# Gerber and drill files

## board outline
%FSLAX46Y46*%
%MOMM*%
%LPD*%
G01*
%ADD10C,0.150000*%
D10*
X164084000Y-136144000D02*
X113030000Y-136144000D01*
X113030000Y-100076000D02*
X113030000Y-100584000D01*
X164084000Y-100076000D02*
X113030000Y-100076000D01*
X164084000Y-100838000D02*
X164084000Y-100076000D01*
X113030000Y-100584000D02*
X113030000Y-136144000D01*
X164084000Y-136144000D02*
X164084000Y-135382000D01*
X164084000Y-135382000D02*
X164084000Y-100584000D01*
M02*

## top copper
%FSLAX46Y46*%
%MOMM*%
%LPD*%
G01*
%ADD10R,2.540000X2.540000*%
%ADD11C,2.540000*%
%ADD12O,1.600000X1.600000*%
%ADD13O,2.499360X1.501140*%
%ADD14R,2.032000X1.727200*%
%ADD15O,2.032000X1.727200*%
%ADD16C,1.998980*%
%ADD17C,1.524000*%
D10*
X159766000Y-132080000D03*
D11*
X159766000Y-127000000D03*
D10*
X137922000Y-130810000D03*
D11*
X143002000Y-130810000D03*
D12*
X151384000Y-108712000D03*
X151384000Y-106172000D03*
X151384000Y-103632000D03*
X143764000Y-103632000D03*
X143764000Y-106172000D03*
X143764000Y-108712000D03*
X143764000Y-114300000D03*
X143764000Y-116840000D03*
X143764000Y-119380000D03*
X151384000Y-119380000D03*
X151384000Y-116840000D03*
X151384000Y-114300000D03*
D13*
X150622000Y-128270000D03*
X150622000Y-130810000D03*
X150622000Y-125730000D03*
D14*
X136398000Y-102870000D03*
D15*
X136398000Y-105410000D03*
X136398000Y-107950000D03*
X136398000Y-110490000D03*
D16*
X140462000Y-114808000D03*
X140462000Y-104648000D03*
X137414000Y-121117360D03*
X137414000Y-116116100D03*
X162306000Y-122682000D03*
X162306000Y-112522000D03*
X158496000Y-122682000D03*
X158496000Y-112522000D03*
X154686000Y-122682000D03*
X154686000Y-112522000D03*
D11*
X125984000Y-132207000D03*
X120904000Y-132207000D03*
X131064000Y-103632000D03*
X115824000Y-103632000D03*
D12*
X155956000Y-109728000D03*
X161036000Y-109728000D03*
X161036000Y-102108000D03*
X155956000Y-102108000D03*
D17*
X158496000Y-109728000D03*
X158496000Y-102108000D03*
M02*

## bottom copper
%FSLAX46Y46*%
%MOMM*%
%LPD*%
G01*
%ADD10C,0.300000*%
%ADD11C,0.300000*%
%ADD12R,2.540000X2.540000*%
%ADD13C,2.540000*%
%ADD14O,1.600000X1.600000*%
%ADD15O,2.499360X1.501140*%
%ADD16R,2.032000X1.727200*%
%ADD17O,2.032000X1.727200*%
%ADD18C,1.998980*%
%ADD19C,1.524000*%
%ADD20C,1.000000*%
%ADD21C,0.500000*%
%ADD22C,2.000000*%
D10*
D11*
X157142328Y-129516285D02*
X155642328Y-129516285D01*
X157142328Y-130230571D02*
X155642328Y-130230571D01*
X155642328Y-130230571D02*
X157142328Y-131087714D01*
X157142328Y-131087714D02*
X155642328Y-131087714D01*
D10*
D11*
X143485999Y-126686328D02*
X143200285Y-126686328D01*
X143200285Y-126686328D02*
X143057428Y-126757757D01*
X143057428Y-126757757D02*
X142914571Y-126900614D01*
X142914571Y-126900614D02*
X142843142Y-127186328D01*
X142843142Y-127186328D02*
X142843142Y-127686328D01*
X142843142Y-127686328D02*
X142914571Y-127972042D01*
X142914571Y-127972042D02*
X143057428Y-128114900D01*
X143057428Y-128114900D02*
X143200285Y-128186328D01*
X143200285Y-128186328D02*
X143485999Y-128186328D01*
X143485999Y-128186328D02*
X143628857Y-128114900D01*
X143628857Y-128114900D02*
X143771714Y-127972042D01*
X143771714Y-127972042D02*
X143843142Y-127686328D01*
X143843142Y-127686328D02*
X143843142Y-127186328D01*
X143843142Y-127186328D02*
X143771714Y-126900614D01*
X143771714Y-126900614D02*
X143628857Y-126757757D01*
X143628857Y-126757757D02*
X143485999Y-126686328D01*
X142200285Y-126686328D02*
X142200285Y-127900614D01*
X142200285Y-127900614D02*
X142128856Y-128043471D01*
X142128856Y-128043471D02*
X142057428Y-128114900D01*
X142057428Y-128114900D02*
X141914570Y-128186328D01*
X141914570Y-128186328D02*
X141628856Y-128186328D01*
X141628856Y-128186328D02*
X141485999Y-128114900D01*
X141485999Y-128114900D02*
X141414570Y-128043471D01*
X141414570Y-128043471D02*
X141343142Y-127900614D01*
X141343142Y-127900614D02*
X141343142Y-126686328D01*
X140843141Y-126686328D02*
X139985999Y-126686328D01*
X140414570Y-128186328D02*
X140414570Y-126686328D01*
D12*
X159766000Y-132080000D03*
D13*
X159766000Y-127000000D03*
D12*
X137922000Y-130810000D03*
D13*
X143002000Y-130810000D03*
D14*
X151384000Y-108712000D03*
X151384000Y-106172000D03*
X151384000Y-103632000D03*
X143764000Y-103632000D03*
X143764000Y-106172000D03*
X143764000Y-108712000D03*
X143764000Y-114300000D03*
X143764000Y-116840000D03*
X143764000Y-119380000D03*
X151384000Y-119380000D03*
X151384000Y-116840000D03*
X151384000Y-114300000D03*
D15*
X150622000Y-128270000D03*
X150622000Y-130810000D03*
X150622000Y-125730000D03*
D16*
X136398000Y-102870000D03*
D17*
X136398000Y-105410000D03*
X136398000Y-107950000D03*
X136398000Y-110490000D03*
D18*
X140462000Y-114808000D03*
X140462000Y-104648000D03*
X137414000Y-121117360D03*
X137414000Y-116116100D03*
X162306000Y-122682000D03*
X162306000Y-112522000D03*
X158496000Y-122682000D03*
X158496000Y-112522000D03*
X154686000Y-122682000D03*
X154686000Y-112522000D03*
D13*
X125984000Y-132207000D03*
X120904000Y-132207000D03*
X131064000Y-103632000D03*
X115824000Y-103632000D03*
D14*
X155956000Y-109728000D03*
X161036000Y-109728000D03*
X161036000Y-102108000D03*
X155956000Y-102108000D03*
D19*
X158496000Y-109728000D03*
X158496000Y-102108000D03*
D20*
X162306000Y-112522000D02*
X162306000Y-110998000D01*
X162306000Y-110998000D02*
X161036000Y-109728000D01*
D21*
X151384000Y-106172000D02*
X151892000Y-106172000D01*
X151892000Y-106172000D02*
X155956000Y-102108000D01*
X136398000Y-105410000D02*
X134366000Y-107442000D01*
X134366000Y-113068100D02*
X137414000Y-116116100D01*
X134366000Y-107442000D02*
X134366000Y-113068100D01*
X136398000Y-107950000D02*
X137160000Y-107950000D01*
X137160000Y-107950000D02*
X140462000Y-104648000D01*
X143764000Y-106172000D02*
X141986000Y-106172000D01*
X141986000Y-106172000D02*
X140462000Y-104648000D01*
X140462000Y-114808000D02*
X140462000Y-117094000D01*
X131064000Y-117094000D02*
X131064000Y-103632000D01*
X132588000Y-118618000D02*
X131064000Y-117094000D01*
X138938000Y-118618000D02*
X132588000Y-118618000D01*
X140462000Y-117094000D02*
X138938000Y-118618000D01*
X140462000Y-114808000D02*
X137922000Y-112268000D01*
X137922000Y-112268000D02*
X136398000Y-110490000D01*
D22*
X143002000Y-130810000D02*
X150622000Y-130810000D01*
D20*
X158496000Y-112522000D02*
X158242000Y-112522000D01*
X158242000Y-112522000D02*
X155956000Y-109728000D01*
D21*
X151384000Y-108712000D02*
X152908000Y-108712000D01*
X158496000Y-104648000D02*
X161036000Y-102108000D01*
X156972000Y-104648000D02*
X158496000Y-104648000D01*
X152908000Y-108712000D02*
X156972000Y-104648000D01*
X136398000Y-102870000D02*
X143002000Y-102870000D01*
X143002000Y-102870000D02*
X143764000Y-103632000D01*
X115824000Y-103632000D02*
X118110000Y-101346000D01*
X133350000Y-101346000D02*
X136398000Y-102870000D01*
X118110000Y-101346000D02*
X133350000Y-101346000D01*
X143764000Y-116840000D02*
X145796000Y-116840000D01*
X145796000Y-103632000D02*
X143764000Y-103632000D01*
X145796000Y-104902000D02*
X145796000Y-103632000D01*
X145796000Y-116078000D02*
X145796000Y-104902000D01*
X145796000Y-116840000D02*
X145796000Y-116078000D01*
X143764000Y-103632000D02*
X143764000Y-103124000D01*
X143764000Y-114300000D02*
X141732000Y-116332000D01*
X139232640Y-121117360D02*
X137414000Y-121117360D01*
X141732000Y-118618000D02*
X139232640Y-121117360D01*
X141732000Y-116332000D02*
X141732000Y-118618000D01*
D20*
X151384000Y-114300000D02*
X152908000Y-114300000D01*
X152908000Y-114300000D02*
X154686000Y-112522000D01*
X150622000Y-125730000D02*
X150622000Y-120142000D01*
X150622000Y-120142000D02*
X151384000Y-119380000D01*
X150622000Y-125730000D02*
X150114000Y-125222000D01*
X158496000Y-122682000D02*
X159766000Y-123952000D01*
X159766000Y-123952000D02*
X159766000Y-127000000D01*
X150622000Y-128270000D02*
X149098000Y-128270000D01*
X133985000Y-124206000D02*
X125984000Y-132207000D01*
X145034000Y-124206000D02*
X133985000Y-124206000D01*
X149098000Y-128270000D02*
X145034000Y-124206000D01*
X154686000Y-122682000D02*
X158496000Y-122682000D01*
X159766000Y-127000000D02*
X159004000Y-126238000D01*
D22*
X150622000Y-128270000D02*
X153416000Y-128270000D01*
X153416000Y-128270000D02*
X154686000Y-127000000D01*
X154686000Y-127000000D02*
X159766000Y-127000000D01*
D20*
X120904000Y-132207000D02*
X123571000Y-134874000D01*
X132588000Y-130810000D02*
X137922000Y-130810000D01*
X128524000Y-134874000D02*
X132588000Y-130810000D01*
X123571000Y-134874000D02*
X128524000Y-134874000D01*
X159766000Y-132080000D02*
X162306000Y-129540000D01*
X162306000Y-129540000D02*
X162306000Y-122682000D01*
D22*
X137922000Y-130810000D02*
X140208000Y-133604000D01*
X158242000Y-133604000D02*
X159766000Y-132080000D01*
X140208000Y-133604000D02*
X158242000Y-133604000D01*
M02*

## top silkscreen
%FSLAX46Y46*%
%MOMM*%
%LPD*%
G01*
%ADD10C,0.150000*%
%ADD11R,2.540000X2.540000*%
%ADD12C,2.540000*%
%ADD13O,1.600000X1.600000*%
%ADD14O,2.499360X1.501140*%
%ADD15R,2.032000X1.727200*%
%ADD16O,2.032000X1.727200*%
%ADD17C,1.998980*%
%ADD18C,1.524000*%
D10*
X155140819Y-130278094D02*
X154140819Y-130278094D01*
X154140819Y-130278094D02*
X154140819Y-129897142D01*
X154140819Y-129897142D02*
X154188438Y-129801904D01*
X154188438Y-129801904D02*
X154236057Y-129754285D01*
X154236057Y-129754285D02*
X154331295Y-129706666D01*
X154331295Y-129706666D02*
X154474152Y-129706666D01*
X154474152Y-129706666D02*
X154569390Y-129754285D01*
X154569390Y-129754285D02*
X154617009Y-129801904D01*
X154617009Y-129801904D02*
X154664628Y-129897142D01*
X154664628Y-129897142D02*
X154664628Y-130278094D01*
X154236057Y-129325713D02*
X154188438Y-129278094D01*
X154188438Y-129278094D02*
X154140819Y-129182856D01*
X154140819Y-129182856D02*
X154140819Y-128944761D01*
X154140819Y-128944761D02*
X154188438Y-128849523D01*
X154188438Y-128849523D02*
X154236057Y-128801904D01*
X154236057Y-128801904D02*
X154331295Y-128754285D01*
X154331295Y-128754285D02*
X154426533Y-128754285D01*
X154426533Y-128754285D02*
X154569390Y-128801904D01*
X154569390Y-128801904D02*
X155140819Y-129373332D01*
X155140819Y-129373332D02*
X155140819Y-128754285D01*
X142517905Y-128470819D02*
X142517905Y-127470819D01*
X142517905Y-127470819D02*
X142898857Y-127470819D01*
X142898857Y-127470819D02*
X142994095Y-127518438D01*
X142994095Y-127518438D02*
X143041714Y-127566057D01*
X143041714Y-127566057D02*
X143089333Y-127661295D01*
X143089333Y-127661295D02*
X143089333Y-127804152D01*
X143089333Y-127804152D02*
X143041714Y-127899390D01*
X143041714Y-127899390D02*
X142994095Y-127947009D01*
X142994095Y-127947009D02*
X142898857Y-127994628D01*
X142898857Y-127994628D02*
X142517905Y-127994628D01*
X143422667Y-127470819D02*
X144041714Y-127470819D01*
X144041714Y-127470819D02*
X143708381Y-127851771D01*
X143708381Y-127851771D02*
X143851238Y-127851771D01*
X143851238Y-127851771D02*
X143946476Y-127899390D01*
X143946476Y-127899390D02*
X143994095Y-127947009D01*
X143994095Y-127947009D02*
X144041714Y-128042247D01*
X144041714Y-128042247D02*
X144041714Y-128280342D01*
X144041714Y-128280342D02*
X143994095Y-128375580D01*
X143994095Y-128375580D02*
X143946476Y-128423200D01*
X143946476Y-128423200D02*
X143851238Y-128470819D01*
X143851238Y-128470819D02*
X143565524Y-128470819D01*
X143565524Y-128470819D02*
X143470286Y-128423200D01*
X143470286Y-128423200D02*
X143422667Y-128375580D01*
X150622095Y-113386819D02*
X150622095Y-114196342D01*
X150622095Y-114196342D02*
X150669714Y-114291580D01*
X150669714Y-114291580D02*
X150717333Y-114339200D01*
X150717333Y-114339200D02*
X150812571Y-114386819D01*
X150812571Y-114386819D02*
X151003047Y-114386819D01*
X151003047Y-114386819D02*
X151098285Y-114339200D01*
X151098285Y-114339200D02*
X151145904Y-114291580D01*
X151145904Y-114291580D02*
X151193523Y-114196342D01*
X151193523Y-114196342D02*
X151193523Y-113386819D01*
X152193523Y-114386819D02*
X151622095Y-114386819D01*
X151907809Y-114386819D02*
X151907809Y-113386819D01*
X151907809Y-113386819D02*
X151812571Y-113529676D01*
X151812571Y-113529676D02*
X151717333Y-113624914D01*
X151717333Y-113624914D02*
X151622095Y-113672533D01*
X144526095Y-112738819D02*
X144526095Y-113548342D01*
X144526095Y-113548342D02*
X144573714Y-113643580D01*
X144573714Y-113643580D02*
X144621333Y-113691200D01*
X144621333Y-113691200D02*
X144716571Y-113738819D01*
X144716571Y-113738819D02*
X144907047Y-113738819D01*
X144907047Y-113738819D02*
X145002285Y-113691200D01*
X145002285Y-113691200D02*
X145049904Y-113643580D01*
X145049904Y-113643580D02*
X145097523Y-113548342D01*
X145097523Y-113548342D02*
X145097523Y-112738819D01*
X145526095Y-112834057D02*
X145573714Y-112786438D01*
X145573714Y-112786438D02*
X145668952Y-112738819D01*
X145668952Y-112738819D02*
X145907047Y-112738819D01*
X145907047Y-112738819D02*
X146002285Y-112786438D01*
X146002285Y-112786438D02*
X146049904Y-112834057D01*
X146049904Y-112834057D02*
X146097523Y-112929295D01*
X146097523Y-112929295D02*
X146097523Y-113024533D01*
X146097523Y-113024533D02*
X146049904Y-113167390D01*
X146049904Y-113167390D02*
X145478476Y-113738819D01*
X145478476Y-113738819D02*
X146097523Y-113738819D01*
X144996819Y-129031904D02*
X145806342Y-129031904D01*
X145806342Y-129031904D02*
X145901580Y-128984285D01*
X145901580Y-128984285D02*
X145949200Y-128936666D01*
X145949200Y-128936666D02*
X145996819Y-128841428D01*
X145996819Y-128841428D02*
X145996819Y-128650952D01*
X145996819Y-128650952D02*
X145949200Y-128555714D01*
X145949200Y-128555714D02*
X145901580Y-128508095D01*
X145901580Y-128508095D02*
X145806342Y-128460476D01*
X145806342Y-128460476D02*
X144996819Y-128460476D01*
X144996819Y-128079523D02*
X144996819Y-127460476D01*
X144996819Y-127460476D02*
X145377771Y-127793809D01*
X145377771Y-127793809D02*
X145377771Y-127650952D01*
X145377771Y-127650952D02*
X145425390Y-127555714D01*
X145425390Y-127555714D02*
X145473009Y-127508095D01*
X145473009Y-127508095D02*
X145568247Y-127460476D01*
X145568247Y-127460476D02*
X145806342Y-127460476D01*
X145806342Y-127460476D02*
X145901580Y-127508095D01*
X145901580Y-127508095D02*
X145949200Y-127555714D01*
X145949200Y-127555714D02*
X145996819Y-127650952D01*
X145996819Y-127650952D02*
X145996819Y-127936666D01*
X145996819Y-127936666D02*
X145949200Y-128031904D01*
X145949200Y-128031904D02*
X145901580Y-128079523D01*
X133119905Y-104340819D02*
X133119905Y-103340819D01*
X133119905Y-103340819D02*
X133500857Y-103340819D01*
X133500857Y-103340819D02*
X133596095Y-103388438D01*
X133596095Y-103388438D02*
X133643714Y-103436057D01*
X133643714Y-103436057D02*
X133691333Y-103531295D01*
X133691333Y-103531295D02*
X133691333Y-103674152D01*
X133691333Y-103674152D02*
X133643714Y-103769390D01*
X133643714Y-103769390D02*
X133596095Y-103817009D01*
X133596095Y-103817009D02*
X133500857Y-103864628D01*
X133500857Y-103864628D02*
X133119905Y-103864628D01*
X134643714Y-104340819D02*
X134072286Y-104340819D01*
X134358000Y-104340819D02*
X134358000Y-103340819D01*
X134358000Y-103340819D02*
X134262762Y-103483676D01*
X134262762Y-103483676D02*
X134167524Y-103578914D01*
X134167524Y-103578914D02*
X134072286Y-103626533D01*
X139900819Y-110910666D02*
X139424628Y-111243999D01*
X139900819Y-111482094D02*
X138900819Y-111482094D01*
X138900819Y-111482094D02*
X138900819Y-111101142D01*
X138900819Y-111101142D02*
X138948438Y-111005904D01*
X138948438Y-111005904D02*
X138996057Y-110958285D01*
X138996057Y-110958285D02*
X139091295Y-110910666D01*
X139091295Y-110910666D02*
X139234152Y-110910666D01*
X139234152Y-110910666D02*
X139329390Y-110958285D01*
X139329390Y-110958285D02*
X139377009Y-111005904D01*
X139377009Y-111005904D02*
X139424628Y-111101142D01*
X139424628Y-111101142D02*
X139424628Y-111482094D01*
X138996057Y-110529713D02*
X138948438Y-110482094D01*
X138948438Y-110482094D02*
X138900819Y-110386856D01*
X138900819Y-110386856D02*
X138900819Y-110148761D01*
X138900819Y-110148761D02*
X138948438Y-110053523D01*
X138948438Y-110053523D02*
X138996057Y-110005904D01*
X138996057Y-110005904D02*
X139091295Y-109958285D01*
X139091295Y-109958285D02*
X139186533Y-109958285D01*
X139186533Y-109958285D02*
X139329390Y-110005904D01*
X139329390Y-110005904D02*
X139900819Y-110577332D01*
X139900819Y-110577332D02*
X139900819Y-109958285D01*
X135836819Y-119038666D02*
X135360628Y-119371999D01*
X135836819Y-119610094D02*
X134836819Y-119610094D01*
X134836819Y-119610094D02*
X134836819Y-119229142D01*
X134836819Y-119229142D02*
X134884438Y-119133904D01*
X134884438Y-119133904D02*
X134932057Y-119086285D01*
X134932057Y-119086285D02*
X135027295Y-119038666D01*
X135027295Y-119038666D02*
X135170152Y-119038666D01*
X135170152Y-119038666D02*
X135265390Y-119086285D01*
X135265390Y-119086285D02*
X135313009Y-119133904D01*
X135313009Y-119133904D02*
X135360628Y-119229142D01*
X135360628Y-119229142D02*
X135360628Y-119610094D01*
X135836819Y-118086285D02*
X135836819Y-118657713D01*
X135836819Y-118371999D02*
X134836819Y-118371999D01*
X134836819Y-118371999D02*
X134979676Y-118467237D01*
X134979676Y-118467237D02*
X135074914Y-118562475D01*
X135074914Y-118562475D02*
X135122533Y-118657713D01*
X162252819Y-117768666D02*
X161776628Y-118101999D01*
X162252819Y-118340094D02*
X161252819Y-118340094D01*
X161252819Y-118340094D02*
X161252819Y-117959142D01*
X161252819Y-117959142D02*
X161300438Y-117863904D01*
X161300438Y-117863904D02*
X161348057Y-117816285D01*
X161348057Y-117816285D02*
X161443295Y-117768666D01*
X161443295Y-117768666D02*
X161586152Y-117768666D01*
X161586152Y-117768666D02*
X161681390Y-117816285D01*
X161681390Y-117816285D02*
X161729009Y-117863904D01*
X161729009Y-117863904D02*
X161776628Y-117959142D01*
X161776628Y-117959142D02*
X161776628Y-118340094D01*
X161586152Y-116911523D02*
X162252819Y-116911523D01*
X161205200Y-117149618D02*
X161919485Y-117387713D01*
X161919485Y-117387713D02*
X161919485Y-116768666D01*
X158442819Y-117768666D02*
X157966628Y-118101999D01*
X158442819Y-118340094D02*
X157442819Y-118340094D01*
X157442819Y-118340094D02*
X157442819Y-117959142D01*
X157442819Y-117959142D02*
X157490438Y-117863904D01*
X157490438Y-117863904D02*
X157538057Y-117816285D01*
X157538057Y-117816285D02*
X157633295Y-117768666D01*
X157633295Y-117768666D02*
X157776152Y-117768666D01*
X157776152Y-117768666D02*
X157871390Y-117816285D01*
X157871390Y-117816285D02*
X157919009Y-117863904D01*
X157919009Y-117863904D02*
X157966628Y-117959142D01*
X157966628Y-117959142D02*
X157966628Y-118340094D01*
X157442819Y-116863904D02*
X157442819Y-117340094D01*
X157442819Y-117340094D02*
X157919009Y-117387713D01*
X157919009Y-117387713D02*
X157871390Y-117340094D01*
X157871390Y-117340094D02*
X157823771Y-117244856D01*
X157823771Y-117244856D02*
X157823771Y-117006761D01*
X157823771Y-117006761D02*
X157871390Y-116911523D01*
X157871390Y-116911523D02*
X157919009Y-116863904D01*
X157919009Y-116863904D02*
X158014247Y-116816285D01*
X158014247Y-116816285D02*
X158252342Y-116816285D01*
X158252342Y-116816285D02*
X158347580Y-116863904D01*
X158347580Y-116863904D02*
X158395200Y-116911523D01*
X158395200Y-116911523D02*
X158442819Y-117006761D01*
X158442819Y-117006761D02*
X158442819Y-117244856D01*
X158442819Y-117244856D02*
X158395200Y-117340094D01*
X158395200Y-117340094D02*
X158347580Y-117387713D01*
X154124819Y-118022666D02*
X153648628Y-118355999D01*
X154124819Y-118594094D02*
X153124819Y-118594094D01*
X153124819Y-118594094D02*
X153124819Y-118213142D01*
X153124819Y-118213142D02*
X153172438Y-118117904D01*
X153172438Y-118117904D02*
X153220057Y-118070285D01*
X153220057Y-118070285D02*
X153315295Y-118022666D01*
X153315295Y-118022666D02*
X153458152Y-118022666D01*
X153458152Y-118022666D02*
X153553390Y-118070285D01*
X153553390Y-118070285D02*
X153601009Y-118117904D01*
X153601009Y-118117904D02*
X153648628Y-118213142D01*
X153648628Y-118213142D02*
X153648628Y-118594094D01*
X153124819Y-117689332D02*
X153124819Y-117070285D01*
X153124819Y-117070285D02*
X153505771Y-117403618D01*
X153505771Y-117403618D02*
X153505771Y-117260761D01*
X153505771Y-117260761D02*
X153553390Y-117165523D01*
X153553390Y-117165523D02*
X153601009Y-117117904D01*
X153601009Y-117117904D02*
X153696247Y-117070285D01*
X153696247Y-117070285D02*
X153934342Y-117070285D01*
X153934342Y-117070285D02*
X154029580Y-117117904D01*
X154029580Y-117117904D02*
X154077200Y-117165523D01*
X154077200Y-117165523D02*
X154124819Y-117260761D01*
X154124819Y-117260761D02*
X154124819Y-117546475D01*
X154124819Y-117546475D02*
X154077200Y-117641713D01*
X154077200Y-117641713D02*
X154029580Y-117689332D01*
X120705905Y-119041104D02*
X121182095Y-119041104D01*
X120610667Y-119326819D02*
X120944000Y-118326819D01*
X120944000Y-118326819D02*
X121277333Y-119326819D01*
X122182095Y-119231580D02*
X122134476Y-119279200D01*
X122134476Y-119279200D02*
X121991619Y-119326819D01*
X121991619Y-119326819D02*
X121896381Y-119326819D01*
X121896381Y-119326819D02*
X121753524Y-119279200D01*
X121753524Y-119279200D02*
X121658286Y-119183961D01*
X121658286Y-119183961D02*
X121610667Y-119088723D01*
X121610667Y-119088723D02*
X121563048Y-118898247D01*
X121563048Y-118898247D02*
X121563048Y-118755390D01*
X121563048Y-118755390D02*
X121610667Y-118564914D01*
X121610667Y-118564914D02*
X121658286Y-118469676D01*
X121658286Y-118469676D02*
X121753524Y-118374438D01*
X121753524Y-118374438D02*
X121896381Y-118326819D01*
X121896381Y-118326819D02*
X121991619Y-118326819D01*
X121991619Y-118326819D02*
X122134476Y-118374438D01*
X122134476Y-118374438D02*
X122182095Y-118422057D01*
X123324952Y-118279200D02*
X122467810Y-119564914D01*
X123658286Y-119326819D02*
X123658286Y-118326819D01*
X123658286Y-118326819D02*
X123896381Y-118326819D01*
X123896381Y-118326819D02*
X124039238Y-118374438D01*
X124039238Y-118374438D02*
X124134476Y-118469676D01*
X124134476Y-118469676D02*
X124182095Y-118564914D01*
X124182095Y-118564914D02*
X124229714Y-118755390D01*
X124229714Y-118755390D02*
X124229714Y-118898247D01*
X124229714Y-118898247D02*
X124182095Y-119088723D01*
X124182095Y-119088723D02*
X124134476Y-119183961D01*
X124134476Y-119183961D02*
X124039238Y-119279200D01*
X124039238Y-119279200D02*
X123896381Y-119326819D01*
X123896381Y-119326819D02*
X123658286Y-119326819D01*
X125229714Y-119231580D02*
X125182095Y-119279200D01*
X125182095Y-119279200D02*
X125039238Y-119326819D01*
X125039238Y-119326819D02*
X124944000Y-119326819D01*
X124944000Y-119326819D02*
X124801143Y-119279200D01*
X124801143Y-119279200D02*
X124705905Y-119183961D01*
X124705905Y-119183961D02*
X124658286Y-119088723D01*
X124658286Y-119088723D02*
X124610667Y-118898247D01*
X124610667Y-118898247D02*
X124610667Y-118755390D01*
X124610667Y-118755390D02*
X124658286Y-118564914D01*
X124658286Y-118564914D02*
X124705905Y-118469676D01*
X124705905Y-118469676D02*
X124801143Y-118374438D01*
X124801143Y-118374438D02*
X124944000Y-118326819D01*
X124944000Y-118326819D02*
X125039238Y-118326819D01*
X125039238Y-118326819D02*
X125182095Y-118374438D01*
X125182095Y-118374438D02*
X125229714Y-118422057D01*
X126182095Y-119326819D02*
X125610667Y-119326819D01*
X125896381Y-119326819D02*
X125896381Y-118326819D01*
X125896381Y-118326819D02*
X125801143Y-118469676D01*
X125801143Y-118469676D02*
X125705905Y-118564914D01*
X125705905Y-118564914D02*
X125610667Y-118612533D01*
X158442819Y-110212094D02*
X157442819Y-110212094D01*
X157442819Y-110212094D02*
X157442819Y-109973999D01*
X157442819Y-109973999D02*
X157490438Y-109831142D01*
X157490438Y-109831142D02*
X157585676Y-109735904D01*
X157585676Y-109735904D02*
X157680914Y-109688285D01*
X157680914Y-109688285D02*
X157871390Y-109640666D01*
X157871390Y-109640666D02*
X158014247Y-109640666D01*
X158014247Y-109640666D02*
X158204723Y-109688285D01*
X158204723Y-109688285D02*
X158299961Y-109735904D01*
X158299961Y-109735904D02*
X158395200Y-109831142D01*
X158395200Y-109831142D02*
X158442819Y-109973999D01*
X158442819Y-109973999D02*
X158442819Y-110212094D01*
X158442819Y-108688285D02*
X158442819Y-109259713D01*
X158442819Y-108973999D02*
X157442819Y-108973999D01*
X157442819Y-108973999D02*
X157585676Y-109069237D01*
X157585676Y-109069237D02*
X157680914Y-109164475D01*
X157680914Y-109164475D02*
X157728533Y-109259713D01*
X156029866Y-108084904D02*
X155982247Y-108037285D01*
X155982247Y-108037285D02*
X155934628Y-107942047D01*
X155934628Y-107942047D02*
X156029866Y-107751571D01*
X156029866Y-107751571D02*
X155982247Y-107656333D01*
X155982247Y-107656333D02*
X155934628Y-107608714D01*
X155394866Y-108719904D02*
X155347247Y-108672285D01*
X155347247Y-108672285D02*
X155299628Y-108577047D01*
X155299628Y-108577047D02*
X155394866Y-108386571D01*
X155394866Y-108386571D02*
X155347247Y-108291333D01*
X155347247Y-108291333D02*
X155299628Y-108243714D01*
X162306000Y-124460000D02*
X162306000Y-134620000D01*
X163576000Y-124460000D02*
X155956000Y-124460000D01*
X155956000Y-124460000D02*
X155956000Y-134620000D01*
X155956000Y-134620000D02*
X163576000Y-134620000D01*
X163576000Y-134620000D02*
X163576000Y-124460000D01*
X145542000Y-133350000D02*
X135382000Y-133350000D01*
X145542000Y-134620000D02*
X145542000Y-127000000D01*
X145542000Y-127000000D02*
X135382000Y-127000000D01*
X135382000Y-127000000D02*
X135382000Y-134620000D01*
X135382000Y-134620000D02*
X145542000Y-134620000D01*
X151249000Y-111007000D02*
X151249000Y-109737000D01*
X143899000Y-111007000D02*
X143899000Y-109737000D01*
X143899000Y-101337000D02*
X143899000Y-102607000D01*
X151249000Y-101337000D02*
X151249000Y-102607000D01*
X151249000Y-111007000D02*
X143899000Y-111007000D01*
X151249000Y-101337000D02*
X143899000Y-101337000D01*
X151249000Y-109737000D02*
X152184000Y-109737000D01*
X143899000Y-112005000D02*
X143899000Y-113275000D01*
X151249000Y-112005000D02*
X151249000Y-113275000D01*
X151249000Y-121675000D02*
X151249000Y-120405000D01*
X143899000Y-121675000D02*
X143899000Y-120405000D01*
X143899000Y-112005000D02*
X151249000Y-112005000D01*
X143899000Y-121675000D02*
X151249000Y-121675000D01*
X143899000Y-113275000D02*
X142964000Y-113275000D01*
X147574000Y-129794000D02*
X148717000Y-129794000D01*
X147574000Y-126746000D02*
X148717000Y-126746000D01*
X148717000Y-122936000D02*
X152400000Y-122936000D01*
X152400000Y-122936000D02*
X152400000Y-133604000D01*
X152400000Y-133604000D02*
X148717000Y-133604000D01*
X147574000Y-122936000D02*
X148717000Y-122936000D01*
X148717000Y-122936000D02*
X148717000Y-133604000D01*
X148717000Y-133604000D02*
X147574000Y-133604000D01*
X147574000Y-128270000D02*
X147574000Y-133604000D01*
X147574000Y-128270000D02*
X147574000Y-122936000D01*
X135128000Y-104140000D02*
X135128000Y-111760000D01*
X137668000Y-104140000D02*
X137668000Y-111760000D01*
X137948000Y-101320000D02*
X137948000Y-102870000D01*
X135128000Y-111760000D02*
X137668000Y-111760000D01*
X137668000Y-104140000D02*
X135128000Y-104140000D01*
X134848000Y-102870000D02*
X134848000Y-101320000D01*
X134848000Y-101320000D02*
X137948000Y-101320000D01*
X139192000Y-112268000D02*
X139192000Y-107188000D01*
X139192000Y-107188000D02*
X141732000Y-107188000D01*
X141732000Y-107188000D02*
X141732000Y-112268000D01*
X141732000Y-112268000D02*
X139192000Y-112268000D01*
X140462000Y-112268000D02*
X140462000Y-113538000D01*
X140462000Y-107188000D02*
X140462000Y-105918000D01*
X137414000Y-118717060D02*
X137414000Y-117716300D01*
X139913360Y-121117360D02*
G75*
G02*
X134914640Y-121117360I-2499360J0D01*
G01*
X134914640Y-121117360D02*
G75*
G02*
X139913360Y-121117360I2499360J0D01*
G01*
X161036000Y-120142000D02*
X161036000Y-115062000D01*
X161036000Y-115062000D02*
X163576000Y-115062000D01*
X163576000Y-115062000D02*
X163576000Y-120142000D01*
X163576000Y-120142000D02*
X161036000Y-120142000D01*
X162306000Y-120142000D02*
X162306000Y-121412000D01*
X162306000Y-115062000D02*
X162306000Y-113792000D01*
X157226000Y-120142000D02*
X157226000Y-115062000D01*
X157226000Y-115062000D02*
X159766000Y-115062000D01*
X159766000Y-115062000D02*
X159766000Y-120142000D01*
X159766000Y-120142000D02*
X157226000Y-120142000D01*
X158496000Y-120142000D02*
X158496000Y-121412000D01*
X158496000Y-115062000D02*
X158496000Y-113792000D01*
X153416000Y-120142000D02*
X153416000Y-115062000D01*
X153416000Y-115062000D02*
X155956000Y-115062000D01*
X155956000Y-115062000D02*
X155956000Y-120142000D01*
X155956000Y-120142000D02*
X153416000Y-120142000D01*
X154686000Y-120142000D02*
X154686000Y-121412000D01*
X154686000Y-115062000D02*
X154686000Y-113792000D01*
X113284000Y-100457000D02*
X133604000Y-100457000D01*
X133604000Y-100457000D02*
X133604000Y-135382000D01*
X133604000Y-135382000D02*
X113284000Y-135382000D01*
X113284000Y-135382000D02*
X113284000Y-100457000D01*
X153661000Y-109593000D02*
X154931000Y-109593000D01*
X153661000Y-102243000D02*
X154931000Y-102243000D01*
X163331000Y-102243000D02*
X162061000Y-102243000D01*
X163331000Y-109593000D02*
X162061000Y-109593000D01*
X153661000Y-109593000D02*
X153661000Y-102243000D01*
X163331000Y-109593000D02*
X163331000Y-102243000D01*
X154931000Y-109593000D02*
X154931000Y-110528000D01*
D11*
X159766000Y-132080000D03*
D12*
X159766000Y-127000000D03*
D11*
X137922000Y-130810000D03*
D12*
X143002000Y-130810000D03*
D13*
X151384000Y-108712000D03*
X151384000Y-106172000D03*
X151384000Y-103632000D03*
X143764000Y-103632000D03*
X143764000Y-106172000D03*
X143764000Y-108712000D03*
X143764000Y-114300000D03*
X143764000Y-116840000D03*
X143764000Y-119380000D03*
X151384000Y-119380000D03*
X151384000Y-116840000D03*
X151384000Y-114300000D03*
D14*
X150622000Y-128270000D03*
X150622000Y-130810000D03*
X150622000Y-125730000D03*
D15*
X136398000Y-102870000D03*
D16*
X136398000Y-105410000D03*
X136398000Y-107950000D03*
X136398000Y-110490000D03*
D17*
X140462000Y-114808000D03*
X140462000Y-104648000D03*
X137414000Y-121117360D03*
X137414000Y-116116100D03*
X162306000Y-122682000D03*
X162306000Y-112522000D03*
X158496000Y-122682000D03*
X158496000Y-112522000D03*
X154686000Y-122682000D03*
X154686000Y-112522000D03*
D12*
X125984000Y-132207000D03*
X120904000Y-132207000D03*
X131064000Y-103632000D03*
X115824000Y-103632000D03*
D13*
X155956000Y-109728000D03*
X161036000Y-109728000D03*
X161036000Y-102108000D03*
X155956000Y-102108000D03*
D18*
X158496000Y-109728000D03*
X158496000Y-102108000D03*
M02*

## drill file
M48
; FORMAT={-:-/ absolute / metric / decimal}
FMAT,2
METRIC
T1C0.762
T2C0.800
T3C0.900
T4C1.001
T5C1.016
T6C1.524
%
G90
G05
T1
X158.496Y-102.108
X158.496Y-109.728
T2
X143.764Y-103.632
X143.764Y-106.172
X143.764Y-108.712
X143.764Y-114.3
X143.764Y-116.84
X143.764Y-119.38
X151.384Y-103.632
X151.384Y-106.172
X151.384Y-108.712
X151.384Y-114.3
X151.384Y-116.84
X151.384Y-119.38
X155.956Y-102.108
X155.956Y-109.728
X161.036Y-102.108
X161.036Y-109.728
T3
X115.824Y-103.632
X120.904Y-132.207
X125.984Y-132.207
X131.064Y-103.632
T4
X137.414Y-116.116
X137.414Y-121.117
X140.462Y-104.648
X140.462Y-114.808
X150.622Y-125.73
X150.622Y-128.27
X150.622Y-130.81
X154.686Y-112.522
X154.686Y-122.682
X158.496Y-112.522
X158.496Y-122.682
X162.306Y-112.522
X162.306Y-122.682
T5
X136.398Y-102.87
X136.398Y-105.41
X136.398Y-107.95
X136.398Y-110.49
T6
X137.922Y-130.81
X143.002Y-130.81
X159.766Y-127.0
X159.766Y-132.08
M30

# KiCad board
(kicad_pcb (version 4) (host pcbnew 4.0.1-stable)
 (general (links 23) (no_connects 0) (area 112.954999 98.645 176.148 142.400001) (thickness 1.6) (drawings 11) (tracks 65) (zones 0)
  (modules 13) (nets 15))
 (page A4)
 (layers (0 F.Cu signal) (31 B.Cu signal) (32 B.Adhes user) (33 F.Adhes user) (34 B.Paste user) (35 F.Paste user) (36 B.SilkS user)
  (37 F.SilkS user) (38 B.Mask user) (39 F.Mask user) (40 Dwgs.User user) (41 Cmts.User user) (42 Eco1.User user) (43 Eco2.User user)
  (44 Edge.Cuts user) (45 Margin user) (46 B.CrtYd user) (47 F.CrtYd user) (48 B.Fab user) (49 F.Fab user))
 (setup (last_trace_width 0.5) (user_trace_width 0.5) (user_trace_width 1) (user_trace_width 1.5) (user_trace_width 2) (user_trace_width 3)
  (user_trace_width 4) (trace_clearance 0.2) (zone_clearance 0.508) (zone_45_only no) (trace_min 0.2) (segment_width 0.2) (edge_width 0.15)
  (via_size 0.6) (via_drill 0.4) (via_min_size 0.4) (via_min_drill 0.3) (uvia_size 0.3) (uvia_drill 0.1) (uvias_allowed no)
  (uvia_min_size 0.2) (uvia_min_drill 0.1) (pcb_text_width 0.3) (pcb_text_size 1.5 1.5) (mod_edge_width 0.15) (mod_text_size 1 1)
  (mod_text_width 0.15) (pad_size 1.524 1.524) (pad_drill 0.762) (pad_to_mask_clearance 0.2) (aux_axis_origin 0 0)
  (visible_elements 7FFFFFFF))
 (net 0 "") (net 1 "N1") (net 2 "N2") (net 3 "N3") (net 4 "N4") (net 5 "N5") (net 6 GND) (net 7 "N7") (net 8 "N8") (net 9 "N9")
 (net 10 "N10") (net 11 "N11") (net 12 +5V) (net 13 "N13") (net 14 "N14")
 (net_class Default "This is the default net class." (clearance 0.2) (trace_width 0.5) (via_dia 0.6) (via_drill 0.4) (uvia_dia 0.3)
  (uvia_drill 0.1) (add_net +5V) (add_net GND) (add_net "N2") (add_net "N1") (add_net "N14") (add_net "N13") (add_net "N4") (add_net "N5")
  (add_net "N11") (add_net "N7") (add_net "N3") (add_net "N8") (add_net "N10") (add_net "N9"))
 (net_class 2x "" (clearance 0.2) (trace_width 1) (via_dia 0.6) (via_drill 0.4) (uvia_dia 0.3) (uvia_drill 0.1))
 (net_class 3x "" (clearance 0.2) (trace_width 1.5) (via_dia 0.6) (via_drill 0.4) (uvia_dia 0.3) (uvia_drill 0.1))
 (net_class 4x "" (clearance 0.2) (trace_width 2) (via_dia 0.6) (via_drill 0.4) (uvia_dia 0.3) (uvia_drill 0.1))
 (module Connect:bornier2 (layer F.Cu) (at 159.766 129.54 90)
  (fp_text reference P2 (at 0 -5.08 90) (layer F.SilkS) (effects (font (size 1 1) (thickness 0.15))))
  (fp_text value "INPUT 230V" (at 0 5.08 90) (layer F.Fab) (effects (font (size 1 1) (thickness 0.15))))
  (fp_line (start 5.08 2.54) (end -5.08 2.54) (layer F.SilkS) (width 0.15))
  (fp_line (start 5.08 3.81) (end 5.08 -3.81) (layer F.SilkS) (width 0.15))
  (fp_line (start 5.08 -3.81) (end -5.08 -3.81) (layer F.SilkS) (width 0.15))
  (fp_line (start -5.08 -3.81) (end -5.08 3.81) (layer F.SilkS) (width 0.15))
  (fp_line (start -5.08 3.81) (end 5.08 3.81) (layer F.SilkS) (width 0.15))
  (pad 1 thru_hole rect (at -2.54 0 90) (size 2.54 2.54) (drill 1.524) (layers *.Cu *.Mask F.SilkS) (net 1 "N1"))
  (pad 2 thru_hole circle (at 2.54 0 90) (size 2.54 2.54) (drill 1.524) (layers *.Cu *.Mask F.SilkS) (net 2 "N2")))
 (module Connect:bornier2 (layer F.Cu) (at 140.462 130.81)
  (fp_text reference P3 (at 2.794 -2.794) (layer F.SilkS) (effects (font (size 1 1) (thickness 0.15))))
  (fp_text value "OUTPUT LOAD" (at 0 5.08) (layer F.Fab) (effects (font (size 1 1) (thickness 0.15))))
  (fp_line (start 5.08 2.54) (end -5.08 2.54) (layer F.SilkS) (width 0.15))
  (fp_line (start 5.08 3.81) (end 5.08 -3.81) (layer F.SilkS) (width 0.15))
  (fp_line (start 5.08 -3.81) (end -5.08 -3.81) (layer F.SilkS) (width 0.15))
  (fp_line (start -5.08 -3.81) (end -5.08 3.81) (layer F.SilkS) (width 0.15))
  (fp_line (start -5.08 3.81) (end 5.08 3.81) (layer F.SilkS) (width 0.15))
  (pad 1 thru_hole rect (at -2.54 0) (size 2.54 2.54) (drill 1.524) (layers *.Cu *.Mask F.SilkS) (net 1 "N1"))
  (pad 2 thru_hole circle (at 2.54 0) (size 2.54 2.54) (drill 1.524) (layers *.Cu *.Mask F.SilkS) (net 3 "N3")))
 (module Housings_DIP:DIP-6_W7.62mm (layer F.Cu) (at 151.384 108.712 180)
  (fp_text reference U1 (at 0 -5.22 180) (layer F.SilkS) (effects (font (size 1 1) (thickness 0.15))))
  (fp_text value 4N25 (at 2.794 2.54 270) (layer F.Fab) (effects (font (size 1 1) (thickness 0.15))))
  (fp_line (start 0.135 -2.295) (end 0.135 -1.025) (layer F.SilkS) (width 0.15))
  (fp_line (start 7.485 -2.295) (end 7.485 -1.025) (layer F.SilkS) (width 0.15))
  (fp_line (start 7.485 7.375) (end 7.485 6.105) (layer F.SilkS) (width 0.15))
  (fp_line (start 0.135 7.375) (end 0.135 6.105) (layer F.SilkS) (width 0.15))
  (fp_line (start 0.135 -2.295) (end 7.485 -2.295) (layer F.SilkS) (width 0.15))
  (fp_line (start 0.135 7.375) (end 7.485 7.375) (layer F.SilkS) (width 0.15))
  (fp_line (start 0.135 -1.025) (end -0.8 -1.025) (layer F.SilkS) (width 0.15))
  (pad 1 thru_hole oval (at 0 0 180) (size 1.6 1.6) (drill 0.8) (layers *.Cu *.Mask F.SilkS) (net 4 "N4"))
  (pad 2 thru_hole oval (at 0 2.54 180) (size 1.6 1.6) (drill 0.8) (layers *.Cu *.Mask F.SilkS) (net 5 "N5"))
  (pad 3 thru_hole oval (at 0 5.08 180) (size 1.6 1.6) (drill 0.8) (layers *.Cu *.Mask F.SilkS))
  (pad 4 thru_hole oval (at 7.62 5.08 180) (size 1.6 1.6) (drill 0.8) (layers *.Cu *.Mask F.SilkS) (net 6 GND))
  (pad 5 thru_hole oval (at 7.62 2.54 180) (size 1.6 1.6) (drill 0.8) (layers *.Cu *.Mask F.SilkS) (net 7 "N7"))
  (pad 6 thru_hole oval (at 7.62 0 180) (size 1.6 1.6) (drill 0.8) (layers *.Cu *.Mask F.SilkS)))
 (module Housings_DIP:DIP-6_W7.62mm (layer F.Cu) (at 143.764 114.3)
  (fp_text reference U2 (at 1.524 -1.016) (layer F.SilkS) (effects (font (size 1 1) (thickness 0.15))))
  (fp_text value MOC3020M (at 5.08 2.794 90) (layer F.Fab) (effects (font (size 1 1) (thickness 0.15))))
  (fp_line (start 0.135 -2.295) (end 0.135 -1.025) (layer F.SilkS) (width 0.15))
  (fp_line (start 7.485 -2.295) (end 7.485 -1.025) (layer F.SilkS) (width 0.15))
  (fp_line (start 7.485 7.375) (end 7.485 6.105) (layer F.SilkS) (width 0.15))
  (fp_line (start 0.135 7.375) (end 0.135 6.105) (layer F.SilkS) (width 0.15))
  (fp_line (start 0.135 -2.295) (end 7.485 -2.295) (layer F.SilkS) (width 0.15))
  (fp_line (start 0.135 7.375) (end 7.485 7.375) (layer F.SilkS) (width 0.15))
  (fp_line (start 0.135 -1.025) (end -0.8 -1.025) (layer F.SilkS) (width 0.15))
  (pad 1 thru_hole oval (at 0 0) (size 1.6 1.6) (drill 0.8) (layers *.Cu *.Mask F.SilkS) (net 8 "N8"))
  (pad 2 thru_hole oval (at 0 2.54) (size 1.6 1.6) (drill 0.8) (layers *.Cu *.Mask F.SilkS) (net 6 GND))
  (pad 3 thru_hole oval (at 0 5.08) (size 1.6 1.6) (drill 0.8) (layers *.Cu *.Mask F.SilkS))
  (pad 4 thru_hole oval (at 7.62 5.08) (size 1.6 1.6) (drill 0.8) (layers *.Cu *.Mask F.SilkS) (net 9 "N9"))
  (pad 5 thru_hole oval (at 7.62 2.54) (size 1.6 1.6) (drill 0.8) (layers *.Cu *.Mask F.SilkS))
  (pad 6 thru_hole oval (at 7.62 0) (size 1.6 1.6) (drill 0.8) (layers *.Cu *.Mask F.SilkS) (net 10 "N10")))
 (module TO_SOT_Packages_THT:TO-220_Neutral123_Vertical (layer F.Cu) (at 150.622 128.27 90)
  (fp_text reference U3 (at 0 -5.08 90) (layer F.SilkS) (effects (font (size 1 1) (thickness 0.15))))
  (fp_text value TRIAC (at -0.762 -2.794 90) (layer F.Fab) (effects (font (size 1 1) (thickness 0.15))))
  (fp_line (start -1.524 -3.048) (end -1.524 -1.905) (layer F.SilkS) (width 0.15))
  (fp_line (start 1.524 -3.048) (end 1.524 -1.905) (layer F.SilkS) (width 0.15))
  (fp_line (start 5.334 -1.905) (end 5.334 1.778) (layer F.SilkS) (width 0.15))
  (fp_line (start 5.334 1.778) (end -5.334 1.778) (layer F.SilkS) (width 0.15))
  (fp_line (start -5.334 1.778) (end -5.334 -1.905) (layer F.SilkS) (width 0.15))
  (fp_line (start 5.334 -3.048) (end 5.334 -1.905) (layer F.SilkS) (width 0.15))
  (fp_line (start 5.334 -1.905) (end -5.334 -1.905) (layer F.SilkS) (width 0.15))
  (fp_line (start -5.334 -1.905) (end -5.334 -3.048) (layer F.SilkS) (width 0.15))
  (fp_line (start 0 -3.048) (end -5.334 -3.048) (layer F.SilkS) (width 0.15))
  (fp_line (start 0 -3.048) (end 5.334 -3.048) (layer F.SilkS) (width 0.15))
  (pad 2 thru_hole oval (at 0 0 180) (size 2.49936 1.50114) (drill 1.00076) (layers *.Cu *.Mask F.SilkS) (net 2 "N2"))
  (pad 1 thru_hole oval (at -2.54 0 180) (size 2.49936 1.50114) (drill 1.00076) (layers *.Cu *.Mask F.SilkS) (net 3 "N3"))
  (pad 3 thru_hole oval (at 2.54 0 180) (size 2.49936 1.50114) (drill 1.00076) (layers *.Cu *.Mask F.SilkS) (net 9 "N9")))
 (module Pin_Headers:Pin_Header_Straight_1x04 (layer F.Cu) (at 136.398 102.87)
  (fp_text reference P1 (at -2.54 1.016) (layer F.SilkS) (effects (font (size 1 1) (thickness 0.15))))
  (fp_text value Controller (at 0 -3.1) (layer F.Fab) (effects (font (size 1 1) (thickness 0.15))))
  (fp_line (start -1.27 1.27) (end -1.27 8.89) (layer F.SilkS) (width 0.15))
  (fp_line (start 1.27 1.27) (end 1.27 8.89) (layer F.SilkS) (width 0.15))
  (fp_line (start 1.55 -1.55) (end 1.55 0) (layer F.SilkS) (width 0.15))
  (fp_line (start -1.27 8.89) (end 1.27 8.89) (layer F.SilkS) (width 0.15))
  (fp_line (start 1.27 1.27) (end -1.27 1.27) (layer F.SilkS) (width 0.15))
  (fp_line (start -1.55 0) (end -1.55 -1.55) (layer F.SilkS) (width 0.15))
  (fp_line (start -1.55 -1.55) (end 1.55 -1.55) (layer F.SilkS) (width 0.15))
  (pad 1 thru_hole rect (at 0 0) (size 2.032 1.7272) (drill 1.016) (layers *.Cu *.Mask F.SilkS) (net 6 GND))
  (pad 2 thru_hole oval (at 0 2.54) (size 2.032 1.7272) (drill 1.016) (layers *.Cu *.Mask F.SilkS) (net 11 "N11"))
  (pad 3 thru_hole oval (at 0 5.08) (size 2.032 1.7272) (drill 1.016) (layers *.Cu *.Mask F.SilkS) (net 7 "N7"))
  (pad 4 thru_hole oval (at 0 7.62) (size 2.032 1.7272) (drill 1.016) (layers *.Cu *.Mask F.SilkS) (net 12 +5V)))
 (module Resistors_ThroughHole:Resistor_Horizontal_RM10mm (layer F.Cu) (at 140.462 109.728 90)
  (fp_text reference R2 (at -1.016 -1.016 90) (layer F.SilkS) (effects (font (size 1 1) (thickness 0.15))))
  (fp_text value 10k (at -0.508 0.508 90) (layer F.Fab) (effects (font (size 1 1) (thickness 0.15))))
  (fp_line (start -2.54 -1.27) (end 2.54 -1.27) (layer F.SilkS) (width 0.15))
  (fp_line (start 2.54 -1.27) (end 2.54 1.27) (layer F.SilkS) (width 0.15))
  (fp_line (start 2.54 1.27) (end -2.54 1.27) (layer F.SilkS) (width 0.15))
  (fp_line (start -2.54 1.27) (end -2.54 -1.27) (layer F.SilkS) (width 0.15))
  (fp_line (start -2.54 0) (end -3.81 0) (layer F.SilkS) (width 0.15))
  (fp_line (start 2.54 0) (end 3.81 0) (layer F.SilkS) (width 0.15))
  (pad 1 thru_hole circle (at -5.08 0 90) (size 1.99898 1.99898) (drill 1.00076) (layers *.Cu *.SilkS *.Mask) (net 12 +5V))
  (pad 2 thru_hole circle (at 5.08 0 90) (size 1.99898 1.99898) (drill 1.00076) (layers *.Cu *.SilkS *.Mask) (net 7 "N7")))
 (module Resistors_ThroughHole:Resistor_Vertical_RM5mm (layer F.Cu) (at 137.414 118.618 90)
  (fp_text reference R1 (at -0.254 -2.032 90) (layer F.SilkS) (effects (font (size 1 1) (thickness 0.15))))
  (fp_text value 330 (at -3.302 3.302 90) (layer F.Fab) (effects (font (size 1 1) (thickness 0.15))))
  (fp_line (start -0.09906 0) (end 0.9017 0) (layer F.SilkS) (width 0.15))
  (fp_circle (center -2.49936 0) (end 0 0) (layer F.SilkS) (width 0.15))
  (pad 1 thru_hole circle (at -2.49936 0 90) (size 1.99898 1.99898) (drill 1.00076) (layers *.Cu *.SilkS *.Mask) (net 8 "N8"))
  (pad 2 thru_hole circle (at 2.5019 0 90) (size 1.99898 1.99898) (drill 1.00076) (layers *.Cu *.SilkS *.Mask) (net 11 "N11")))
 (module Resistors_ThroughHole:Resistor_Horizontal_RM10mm (layer F.Cu) (at 162.306 117.602 90)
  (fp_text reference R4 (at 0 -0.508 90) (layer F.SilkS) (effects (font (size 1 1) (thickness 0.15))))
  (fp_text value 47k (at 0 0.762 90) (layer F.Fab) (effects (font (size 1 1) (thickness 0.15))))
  (fp_line (start -2.54 -1.27) (end 2.54 -1.27) (layer F.SilkS) (width 0.15))
  (fp_line (start 2.54 -1.27) (end 2.54 1.27) (layer F.SilkS) (width 0.15))
  (fp_line (start 2.54 1.27) (end -2.54 1.27) (layer F.SilkS) (width 0.15))
  (fp_line (start -2.54 1.27) (end -2.54 -1.27) (layer F.SilkS) (width 0.15))
  (fp_line (start -2.54 0) (end -3.81 0) (layer F.SilkS) (width 0.15))
  (fp_line (start 2.54 0) (end 3.81 0) (layer F.SilkS) (width 0.15))
  (pad 1 thru_hole circle (at -5.08 0 90) (size 1.99898 1.99898) (drill 1.00076) (layers *.Cu *.SilkS *.Mask) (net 1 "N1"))
  (pad 2 thru_hole circle (at 5.08 0 90) (size 1.99898 1.99898) (drill 1.00076) (layers *.Cu *.SilkS *.Mask) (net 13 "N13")))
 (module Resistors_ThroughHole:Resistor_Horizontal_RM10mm (layer F.Cu) (at 158.496 117.602 90)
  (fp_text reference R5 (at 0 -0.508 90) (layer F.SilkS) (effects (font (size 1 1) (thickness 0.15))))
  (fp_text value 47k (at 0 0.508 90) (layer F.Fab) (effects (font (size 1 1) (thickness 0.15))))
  (fp_line (start -2.54 -1.27) (end 2.54 -1.27) (layer F.SilkS) (width 0.15))
  (fp_line (start 2.54 -1.27) (end 2.54 1.27) (layer F.SilkS) (width 0.15))
  (fp_line (start 2.54 1.27) (end -2.54 1.27) (layer F.SilkS) (width 0.15))
  (fp_line (start -2.54 1.27) (end -2.54 -1.27) (layer F.SilkS) (width 0.15))
  (fp_line (start -2.54 0) (end -3.81 0) (layer F.SilkS) (width 0.15))
  (fp_line (start 2.54 0) (end 3.81 0) (layer F.SilkS) (width 0.15))
  (pad 1 thru_hole circle (at -5.08 0 90) (size 1.99898 1.99898) (drill 1.00076) (layers *.Cu *.SilkS *.Mask) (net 2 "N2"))
  (pad 2 thru_hole circle (at 5.08 0 90) (size 1.99898 1.99898) (drill 1.00076) (layers *.Cu *.SilkS *.Mask) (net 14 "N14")))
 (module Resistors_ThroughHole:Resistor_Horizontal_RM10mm (layer F.Cu) (at 154.686 117.602 90)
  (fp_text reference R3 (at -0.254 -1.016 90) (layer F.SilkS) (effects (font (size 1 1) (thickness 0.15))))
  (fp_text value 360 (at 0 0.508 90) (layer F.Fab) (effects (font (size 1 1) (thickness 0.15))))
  (fp_line (start -2.54 -1.27) (end 2.54 -1.27) (layer F.SilkS) (width 0.15))
  (fp_line (start 2.54 -1.27) (end 2.54 1.27) (layer F.SilkS) (width 0.15))
  (fp_line (start 2.54 1.27) (end -2.54 1.27) (layer F.SilkS) (width 0.15))
  (fp_line (start -2.54 1.27) (end -2.54 -1.27) (layer F.SilkS) (width 0.15))
  (fp_line (start -2.54 0) (end -3.81 0) (layer F.SilkS) (width 0.15))
  (fp_line (start 2.54 0) (end 3.81 0) (layer F.SilkS) (width 0.15))
  (pad 1 thru_hole circle (at -5.08 0 90) (size 1.99898 1.99898) (drill 1.00076) (layers *.Cu *.SilkS *.Mask) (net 2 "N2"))
  (pad 2 thru_hole circle (at 5.08 0 90) (size 1.99898 1.99898) (drill 1.00076) (layers *.Cu *.SilkS *.Mask) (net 10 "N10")))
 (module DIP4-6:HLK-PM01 (layer F.Cu) (at 123.444 117.602)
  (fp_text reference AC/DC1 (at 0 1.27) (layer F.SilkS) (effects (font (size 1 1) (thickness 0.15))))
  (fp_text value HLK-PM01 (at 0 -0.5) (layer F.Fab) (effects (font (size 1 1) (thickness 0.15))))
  (fp_line (start -10.16 -17.145) (end 10.16 -17.145) (layer F.SilkS) (width 0.15))
  (fp_line (start 10.16 -17.145) (end 10.16 17.78) (layer F.SilkS) (width 0.15))
  (fp_line (start 10.16 17.78) (end -10.16 17.78) (layer F.SilkS) (width 0.15))
  (fp_line (start -10.16 17.78) (end -10.16 -17.145) (layer F.SilkS) (width 0.15))
  (pad 1 thru_hole circle (at 2.54 14.605) (size 2.54 2.54) (drill 0.9) (layers *.Cu *.Mask F.SilkS) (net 2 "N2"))
  (pad 2 thru_hole circle (at -2.54 14.605) (size 2.54 2.54) (drill 0.9) (layers *.Cu *.Mask F.SilkS) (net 1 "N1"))
  (pad 3 thru_hole circle (at 7.62 -13.97) (size 2.54 2.54) (drill 0.9) (layers *.Cu *.Mask F.SilkS) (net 12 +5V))
  (pad 4 thru_hole circle (at -7.62 -13.97) (size 2.54 2.54) (drill 0.9) (layers *.Cu *.Mask F.SilkS) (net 6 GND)))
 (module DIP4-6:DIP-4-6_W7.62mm (layer F.Cu) (at 155.956 109.728 90)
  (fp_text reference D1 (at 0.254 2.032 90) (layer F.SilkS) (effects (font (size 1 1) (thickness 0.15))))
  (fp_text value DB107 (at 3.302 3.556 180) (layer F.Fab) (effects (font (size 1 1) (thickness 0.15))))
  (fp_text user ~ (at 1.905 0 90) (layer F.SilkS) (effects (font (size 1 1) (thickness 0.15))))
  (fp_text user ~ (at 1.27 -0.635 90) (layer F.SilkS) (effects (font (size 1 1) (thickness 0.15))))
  (fp_line (start 0.135 -2.295) (end 0.135 -1.025) (layer F.SilkS) (width 0.15))
  (fp_line (start 7.485 -2.295) (end 7.485 -1.025) (layer F.SilkS) (width 0.15))
  (fp_line (start 7.485 7.375) (end 7.485 6.105) (layer F.SilkS) (width 0.15))
  (fp_line (start 0.135 7.375) (end 0.135 6.105) (layer F.SilkS) (width 0.15))
  (fp_line (start 0.135 -2.295) (end 7.485 -2.295) (layer F.SilkS) (width 0.15))
  (fp_line (start 0.135 7.375) (end 7.485 7.375) (layer F.SilkS) (width 0.15))
  (fp_line (start 0.135 -1.025) (end -0.8 -1.025) (layer F.SilkS) (width 0.15))
  (pad 1 thru_hole oval (at 0 0 90) (size 1.6 1.6) (drill 0.8) (layers *.Cu *.Mask F.SilkS) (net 14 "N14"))
  (pad 2 thru_hole oval (at 0 5.08 90) (size 1.6 1.6) (drill 0.8) (layers *.Cu *.Mask F.SilkS) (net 13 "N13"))
  (pad 3 thru_hole oval (at 7.62 5.08 90) (size 1.6 1.6) (drill 0.8) (layers *.Cu *.Mask F.SilkS) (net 4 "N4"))
  (pad 4 thru_hole oval (at 7.62 0 90) (size 1.6 1.6) (drill 0.8) (layers *.Cu *.Mask F.SilkS) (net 5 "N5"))
  (pad "" thru_hole circle (at 0 2.54 90) (size 1.524 1.524) (drill 0.762) (layers *.Cu *.Mask F.SilkS))
  (pad "" thru_hole circle (at 7.62 2.54 90) (size 1.524 1.524) (drill 0.762) (layers *.Cu *.Mask F.SilkS)))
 (gr_line (start 164.084 136.144) (end 113.03 136.144) (angle 90) (layer Edge.Cuts) (width 0.15))
 (gr_line (start 113.03 100.076) (end 113.03 100.584) (angle 90) (layer Edge.Cuts) (width 0.15))
 (gr_line (start 164.084 100.076) (end 113.03 100.076) (angle 90) (layer Edge.Cuts) (width 0.15))
 (gr_line (start 164.084 100.838) (end 164.084 100.076) (angle 90) (layer Edge.Cuts) (width 0.15))
 (gr_line (start 113.03 100.584) (end 113.03 136.144) (angle 90) (layer Edge.Cuts) (width 0.15))
 (gr_line (start 164.084 136.144) (end 164.084 135.382) (angle 90) (layer Edge.Cuts) (width 0.15))
 (gr_line (start 164.084 135.382) (end 164.084 100.584) (angle 90) (layer Edge.Cuts) (width 0.15))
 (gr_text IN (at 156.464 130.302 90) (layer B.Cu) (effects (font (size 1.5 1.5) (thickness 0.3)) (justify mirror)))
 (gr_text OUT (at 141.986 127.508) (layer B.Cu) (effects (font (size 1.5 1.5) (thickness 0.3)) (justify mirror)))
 (segment (start 162.306 112.522) (end 162.306 110.998) (width 1) (layer B.Cu) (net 13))
 (segment (start 162.306 110.998) (end 161.036 109.728) (width 1) (layer B.Cu) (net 13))
 (segment (start 151.384 106.172) (end 151.892 106.172) (width 0.5) (layer B.Cu) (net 5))
 (segment (start 151.892 106.172) (end 155.956 102.108) (width 0.5) (layer B.Cu) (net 5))
 (segment (start 136.398 105.41) (end 134.366 107.442) (width 0.5) (layer B.Cu) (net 11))
 (segment (start 134.366 113.0681) (end 137.414 116.1161) (width 0.5) (layer B.Cu) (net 11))
 (segment (start 134.366 107.442) (end 134.366 113.0681) (width 0.5) (layer B.Cu) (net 11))
 (segment (start 136.398 107.95) (end 137.16 107.95) (width 0.5) (layer B.Cu) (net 7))
 (segment (start 137.16 107.95) (end 140.462 104.648) (width 0.5) (layer B.Cu) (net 7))
 (segment (start 143.764 106.172) (end 141.986 106.172) (width 0.5) (layer B.Cu) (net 7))
 (segment (start 141.986 106.172) (end 140.462 104.648) (width 0.5) (layer B.Cu) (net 7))
 (segment (start 140.462 114.808) (end 140.462 117.094) (width 0.5) (layer B.Cu) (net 12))
 (segment (start 131.064 117.094) (end 131.064 103.632) (width 0.5) (layer B.Cu) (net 12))
 (segment (start 132.588 118.618) (end 131.064 117.094) (width 0.5) (layer B.Cu) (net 12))
 (segment (start 138.938 118.618) (end 132.588 118.618) (width 0.5) (layer B.Cu) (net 12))
 (segment (start 140.462 117.094) (end 138.938 118.618) (width 0.5) (layer B.Cu) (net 12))
 (segment (start 140.462 114.808) (end 137.922 112.268) (width 0.5) (layer B.Cu) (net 12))
 (segment (start 137.922 112.268) (end 136.398 110.49) (width 0.5) (layer B.Cu) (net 12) (status 20))
 (segment (start 143.002 130.81) (end 150.622 130.81) (width 2) (layer B.Cu) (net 3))
 (segment (start 158.496 112.522) (end 158.242 112.522) (width 1) (layer B.Cu) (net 14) (status 30))
 (segment (start 158.242 112.522) (end 155.956 109.728) (width 1) (layer B.Cu) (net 14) (status 10))
 (segment (start 151.384 108.712) (end 152.908 108.712) (width 0.5) (layer B.Cu) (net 4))
 (segment (start 158.496 104.648) (end 161.036 102.108) (width 0.5) (layer B.Cu) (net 4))
 (segment (start 156.972 104.648) (end 158.496 104.648) (width 0.5) (layer B.Cu) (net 4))
 (segment (start 152.908 108.712) (end 156.972 104.648) (width 0.5) (layer B.Cu) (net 4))
 (segment (start 136.398 102.87) (end 143.002 102.87) (width 0.5) (layer B.Cu) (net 6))
 (segment (start 143.002 102.87) (end 143.764 103.632) (width 0.5) (layer B.Cu) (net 6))
 (segment (start 115.824 103.632) (end 118.11 101.346) (width 0.5) (layer B.Cu) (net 6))
 (segment (start 133.35 101.346) (end 136.398 102.87) (width 0.5) (layer B.Cu) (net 6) (status 20))
 (segment (start 118.11 101.346) (end 133.35 101.346) (width 0.5) (layer B.Cu) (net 6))
 (segment (start 143.764 116.84) (end 145.796 116.84) (width 0.5) (layer B.Cu) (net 6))
 (segment (start 145.796 103.632) (end 143.764 103.632) (width 0.5) (layer B.Cu) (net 6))
 (segment (start 145.796 104.902) (end 145.796 103.632) (width 0.5) (layer B.Cu) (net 6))
 (segment (start 145.796 116.078) (end 145.796 104.902) (width 0.5) (layer B.Cu) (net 6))
 (segment (start 145.796 116.84) (end 145.796 116.078) (width 0.5) (layer B.Cu) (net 6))
 (segment (start 143.764 103.632) (end 143.764 103.124) (width 0.5) (layer B.Cu) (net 6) (status 30))
 (segment (start 143.764 114.3) (end 141.732 116.332) (width 0.5) (layer B.Cu) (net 8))
 (segment (start 139.23264 121.11736) (end 137.414 121.11736) (width 0.5) (layer B.Cu) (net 8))
 (segment (start 141.732 118.618) (end 139.23264 121.11736) (width 0.5) (layer B.Cu) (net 8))
 (segment (start 141.732 116.332) (end 141.732 118.618) (width 0.5) (layer B.Cu) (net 8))
 (segment (start 151.384 114.3) (end 152.908 114.3) (width 1) (layer B.Cu) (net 10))
 (segment (start 152.908 114.3) (end 154.686 112.522) (width 1) (layer B.Cu) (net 10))
 (segment (start 150.622 125.73) (end 150.622 120.142) (width 1) (layer B.Cu) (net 9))
 (segment (start 150.622 120.142) (end 151.384 119.38) (width 1) (layer B.Cu) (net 9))
 (segment (start 150.622 125.73) (end 150.114 125.222) (width 1) (layer B.Cu) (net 9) (status 10))
 (segment (start 158.496 122.682) (end 159.766 123.952) (width 1) (layer B.Cu) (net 2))
 (segment (start 159.766 123.952) (end 159.766 127) (width 1) (layer B.Cu) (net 2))
 (segment (start 150.622 128.27) (end 149.098 128.27) (width 1) (layer B.Cu) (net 2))
 (segment (start 133.985 124.206) (end 125.984 132.207) (width 1) (layer B.Cu) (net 2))
 (segment (start 145.034 124.206) (end 133.985 124.206) (width 1) (layer B.Cu) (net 2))
 (segment (start 149.098 128.27) (end 145.034 124.206) (width 1) (layer B.Cu) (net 2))
 (segment (start 154.686 122.682) (end 158.496 122.682) (width 1) (layer B.Cu) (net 2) (status 20))
 (segment (start 159.766 127) (end 159.004 126.238) (width 1) (layer B.Cu) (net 2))
 (segment (start 150.622 128.27) (end 153.416 128.27) (width 2) (layer B.Cu) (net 2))
 (segment (start 153.416 128.27) (end 154.686 127) (width 2) (layer B.Cu) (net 2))
 (segment (start 154.686 127) (end 159.766 127) (width 2) (layer B.Cu) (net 2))
 (segment (start 120.904 132.207) (end 123.571 134.874) (width 1) (layer B.Cu) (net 1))
 (segment (start 132.588 130.81) (end 137.922 130.81) (width 1) (layer B.Cu) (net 1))
 (segment (start 128.524 134.874) (end 132.588 130.81) (width 1) (layer B.Cu) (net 1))
 (segment (start 123.571 134.874) (end 128.524 134.874) (width 1) (layer B.Cu) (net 1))
 (segment (start 159.766 132.08) (end 162.306 129.54) (width 1) (layer B.Cu) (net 1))
 (segment (start 162.306 129.54) (end 162.306 122.682) (width 1) (layer B.Cu) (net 1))
 (segment (start 137.922 130.81) (end 140.208 133.604) (width 2) (layer B.Cu) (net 1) (status 10))
 (segment (start 158.242 133.604) (end 159.766 132.08) (width 2) (layer B.Cu) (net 1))
 (segment (start 140.208 133.604) (end 158.242 133.604) (width 2) (layer B.Cu) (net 1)))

